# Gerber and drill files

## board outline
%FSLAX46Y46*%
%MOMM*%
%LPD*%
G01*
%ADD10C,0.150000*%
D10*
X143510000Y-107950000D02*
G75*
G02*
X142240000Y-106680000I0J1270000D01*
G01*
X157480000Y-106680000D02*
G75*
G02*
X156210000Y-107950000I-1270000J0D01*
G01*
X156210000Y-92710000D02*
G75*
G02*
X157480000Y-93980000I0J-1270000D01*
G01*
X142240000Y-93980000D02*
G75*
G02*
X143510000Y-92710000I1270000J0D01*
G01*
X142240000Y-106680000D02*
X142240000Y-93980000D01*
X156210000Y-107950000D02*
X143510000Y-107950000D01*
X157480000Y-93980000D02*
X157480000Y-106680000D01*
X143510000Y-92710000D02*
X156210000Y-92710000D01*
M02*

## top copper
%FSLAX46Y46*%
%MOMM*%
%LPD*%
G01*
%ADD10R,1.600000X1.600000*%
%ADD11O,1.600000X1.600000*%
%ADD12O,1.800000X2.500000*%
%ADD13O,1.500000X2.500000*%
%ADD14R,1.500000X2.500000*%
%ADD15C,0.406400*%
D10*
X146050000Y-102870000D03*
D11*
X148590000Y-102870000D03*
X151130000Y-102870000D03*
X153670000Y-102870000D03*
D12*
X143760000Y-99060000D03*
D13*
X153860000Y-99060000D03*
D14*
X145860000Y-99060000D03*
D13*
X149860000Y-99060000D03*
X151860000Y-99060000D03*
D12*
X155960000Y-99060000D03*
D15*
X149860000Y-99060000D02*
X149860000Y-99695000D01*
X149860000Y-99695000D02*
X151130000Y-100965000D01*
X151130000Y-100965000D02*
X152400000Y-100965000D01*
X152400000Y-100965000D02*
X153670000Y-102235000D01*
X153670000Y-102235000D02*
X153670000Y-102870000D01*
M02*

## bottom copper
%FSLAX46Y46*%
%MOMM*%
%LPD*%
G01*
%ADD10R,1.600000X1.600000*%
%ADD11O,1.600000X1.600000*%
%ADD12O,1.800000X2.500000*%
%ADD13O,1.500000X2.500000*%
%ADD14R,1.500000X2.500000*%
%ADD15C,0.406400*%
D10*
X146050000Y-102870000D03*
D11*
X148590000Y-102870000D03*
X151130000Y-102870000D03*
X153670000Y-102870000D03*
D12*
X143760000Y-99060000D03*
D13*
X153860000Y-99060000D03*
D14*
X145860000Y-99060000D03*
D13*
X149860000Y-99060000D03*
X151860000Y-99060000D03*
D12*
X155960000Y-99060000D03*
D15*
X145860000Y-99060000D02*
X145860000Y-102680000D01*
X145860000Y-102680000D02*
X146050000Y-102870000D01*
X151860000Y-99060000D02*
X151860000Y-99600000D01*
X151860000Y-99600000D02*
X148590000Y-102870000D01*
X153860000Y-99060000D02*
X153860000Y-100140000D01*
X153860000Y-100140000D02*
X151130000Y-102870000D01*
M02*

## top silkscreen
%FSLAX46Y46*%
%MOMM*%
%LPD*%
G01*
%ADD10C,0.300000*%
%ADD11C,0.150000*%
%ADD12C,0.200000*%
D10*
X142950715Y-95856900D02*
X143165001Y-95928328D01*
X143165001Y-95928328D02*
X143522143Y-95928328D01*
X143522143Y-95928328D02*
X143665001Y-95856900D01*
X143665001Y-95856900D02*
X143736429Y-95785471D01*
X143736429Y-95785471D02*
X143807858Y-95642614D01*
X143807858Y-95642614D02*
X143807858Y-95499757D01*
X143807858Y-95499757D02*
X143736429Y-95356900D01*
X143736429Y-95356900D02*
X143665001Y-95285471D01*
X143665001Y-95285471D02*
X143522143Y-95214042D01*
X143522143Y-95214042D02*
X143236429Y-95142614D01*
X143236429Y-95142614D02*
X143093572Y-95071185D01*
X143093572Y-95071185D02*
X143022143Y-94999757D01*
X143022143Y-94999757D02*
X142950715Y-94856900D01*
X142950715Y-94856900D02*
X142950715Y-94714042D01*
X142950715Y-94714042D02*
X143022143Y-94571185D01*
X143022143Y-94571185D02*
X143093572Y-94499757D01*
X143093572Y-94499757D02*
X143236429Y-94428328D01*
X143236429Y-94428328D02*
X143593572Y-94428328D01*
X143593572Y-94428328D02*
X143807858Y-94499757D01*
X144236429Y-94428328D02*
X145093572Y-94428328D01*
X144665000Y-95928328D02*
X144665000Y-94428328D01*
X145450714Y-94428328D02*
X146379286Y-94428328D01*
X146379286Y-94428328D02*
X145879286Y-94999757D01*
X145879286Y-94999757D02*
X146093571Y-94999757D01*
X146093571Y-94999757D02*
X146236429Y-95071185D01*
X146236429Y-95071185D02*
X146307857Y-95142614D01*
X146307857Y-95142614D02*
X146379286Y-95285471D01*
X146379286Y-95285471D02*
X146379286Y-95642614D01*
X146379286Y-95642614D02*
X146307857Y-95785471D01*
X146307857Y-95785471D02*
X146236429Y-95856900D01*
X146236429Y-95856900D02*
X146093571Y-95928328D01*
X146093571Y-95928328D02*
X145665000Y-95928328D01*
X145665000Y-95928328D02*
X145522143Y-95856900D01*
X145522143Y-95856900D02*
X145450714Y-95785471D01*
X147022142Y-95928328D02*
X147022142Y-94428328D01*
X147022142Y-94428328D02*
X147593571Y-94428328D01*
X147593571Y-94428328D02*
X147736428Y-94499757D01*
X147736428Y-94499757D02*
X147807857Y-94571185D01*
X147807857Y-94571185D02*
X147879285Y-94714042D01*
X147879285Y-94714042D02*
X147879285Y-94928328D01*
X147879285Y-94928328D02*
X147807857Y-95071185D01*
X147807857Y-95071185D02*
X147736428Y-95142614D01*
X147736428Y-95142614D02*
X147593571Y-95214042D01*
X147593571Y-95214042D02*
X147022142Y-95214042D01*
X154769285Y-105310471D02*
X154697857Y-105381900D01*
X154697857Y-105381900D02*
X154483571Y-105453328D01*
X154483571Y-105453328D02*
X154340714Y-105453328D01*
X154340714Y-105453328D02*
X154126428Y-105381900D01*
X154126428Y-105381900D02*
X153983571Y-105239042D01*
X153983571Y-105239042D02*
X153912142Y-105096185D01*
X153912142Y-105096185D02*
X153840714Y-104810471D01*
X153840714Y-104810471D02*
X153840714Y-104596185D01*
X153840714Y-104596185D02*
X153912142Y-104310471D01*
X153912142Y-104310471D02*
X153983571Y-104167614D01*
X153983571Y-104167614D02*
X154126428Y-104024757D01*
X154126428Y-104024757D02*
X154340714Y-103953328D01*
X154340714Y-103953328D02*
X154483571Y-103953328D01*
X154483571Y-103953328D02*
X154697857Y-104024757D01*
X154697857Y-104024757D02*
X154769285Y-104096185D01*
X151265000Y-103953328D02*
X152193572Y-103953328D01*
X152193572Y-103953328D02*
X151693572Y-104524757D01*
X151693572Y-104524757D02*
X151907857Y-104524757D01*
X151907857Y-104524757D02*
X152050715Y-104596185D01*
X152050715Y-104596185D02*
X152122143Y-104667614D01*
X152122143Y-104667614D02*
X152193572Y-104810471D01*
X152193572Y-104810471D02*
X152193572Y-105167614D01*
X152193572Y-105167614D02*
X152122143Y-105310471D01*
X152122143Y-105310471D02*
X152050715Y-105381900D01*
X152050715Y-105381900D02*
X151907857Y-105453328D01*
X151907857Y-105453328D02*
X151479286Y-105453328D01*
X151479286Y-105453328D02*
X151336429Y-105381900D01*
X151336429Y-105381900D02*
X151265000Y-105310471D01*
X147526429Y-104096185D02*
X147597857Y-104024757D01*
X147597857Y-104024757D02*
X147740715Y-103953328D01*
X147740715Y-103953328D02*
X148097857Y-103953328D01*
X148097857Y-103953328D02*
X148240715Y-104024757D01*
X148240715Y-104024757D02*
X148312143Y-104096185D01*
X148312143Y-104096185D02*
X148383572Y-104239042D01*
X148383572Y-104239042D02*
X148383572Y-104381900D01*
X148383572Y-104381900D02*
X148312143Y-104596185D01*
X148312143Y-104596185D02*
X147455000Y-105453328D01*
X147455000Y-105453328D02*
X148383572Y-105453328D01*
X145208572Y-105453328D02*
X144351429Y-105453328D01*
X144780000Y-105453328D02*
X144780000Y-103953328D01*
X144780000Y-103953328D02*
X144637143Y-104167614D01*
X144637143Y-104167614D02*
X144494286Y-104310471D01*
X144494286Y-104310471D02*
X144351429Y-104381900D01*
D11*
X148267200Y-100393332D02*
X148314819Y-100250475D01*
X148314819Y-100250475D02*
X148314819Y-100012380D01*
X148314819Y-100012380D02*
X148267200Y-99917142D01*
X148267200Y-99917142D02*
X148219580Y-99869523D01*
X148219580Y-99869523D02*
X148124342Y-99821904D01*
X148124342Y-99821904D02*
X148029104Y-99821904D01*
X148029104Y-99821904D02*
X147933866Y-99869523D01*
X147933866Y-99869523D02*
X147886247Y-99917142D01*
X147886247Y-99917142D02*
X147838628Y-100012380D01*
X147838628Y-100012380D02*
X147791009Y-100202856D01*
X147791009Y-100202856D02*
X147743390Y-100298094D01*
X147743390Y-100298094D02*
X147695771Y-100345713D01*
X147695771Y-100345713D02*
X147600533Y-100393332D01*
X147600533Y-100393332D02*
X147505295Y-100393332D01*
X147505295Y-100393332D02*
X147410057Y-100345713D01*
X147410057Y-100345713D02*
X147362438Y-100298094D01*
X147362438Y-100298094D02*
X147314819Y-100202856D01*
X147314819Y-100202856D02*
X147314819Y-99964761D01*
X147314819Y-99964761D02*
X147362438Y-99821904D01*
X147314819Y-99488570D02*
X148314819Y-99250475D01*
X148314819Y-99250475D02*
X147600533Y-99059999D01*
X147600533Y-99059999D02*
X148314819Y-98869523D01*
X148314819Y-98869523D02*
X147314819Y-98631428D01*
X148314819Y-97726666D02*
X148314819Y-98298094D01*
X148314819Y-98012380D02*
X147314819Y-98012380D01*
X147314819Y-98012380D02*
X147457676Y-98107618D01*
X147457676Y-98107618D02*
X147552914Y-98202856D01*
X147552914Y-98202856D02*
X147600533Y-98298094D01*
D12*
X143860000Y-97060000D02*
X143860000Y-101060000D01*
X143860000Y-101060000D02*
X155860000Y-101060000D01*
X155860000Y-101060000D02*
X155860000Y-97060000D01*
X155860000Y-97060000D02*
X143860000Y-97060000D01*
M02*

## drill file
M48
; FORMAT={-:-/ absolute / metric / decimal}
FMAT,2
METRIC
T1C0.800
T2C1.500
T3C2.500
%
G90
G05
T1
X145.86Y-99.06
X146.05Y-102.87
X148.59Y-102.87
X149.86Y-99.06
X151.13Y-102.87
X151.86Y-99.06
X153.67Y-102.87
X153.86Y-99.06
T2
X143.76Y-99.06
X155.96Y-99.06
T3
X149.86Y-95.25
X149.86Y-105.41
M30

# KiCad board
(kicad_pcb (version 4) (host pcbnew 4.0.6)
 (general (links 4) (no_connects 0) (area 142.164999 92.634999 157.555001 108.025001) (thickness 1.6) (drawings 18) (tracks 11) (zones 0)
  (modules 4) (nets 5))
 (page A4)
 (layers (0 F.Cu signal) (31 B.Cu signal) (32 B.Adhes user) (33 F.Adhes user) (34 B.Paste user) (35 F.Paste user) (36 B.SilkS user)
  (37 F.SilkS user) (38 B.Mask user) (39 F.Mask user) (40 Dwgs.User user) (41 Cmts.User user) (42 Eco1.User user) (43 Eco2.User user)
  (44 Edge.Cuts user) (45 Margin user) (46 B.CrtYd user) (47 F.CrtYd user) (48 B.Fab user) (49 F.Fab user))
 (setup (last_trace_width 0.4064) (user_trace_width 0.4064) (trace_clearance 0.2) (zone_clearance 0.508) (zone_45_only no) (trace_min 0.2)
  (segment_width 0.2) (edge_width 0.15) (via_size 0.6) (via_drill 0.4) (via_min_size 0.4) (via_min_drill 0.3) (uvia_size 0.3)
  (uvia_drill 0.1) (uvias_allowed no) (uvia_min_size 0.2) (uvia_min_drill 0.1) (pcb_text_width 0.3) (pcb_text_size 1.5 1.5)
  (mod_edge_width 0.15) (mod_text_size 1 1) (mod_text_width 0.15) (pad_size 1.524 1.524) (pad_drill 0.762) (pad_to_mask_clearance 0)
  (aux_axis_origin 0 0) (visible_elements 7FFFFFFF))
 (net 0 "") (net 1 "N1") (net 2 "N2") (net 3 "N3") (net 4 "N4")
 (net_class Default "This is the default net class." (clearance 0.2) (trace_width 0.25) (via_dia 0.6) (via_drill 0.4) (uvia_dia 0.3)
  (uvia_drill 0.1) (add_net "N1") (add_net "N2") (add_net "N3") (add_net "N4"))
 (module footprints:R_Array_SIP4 (layer F.Cu) (at 146.05 102.87)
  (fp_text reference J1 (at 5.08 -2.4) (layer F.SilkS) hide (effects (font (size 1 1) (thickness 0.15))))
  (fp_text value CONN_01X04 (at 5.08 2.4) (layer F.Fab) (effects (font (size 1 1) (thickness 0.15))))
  (pad 1 thru_hole rect (at 0 0) (size 1.6 1.6) (drill 0.8) (layers *.Cu *.Mask) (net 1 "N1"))
  (pad 2 thru_hole oval (at 2.54 0) (size 1.6 1.6) (drill 0.8) (layers *.Cu *.Mask) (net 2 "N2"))
  (pad 3 thru_hole oval (at 5.08 0) (size 1.6 1.6) (drill 0.8) (layers *.Cu *.Mask) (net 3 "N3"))
  (pad 4 thru_hole oval (at 7.62 0) (size 1.6 1.6) (drill 0.8) (layers *.Cu *.Mask) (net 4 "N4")))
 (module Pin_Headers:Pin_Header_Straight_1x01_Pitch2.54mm (layer F.Cu) (at 149.86 105.41)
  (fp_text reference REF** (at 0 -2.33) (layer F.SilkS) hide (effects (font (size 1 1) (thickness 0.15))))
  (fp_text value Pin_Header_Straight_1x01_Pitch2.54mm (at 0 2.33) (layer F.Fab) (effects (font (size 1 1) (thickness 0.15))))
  (pad "" np_thru_hole circle (at 0 0) (size 2.5 2.5) (drill 2.5) (layers *.Cu *.Mask)))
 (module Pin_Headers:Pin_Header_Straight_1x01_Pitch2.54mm (layer F.Cu) (at 149.86 95.25)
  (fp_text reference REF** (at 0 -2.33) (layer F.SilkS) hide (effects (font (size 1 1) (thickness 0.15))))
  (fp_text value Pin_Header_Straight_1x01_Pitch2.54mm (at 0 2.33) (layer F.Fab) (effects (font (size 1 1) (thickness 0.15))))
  (pad "" np_thru_hole circle (at 0 0) (size 2.5 2.5) (drill 2.5) (layers *.Cu *.Mask)))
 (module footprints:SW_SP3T (layer F.Cu) (at 149.86 99.06)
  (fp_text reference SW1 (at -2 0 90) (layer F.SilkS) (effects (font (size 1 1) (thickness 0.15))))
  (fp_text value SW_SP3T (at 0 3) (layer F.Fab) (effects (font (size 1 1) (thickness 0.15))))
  (fp_line (start -6 -2) (end -6 2) (layer F.SilkS) (width 0.2)) (fp_line (start -6 2) (end 6 2) (layer F.SilkS) (width 0.2))
  (fp_line (start 6 2) (end 6 -2) (layer F.SilkS) (width 0.2))
  (fp_line (start 6 -2) (end -6 -2) (layer F.SilkS) (width 0.2))
  (pad 5 thru_hole oval (at -6.1 0) (size 1.8 2.5) (drill 1.5) (layers *.Cu *.Mask))
  (pad 4 thru_hole oval (at 4 0) (size 1.5 2.5) (drill 0.8) (layers *.Cu *.Mask) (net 3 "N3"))
  (pad 1 thru_hole rect (at -4 0) (size 1.5 2.5) (drill 0.8) (layers *.Cu *.Mask) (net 1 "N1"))
  (pad 2 thru_hole oval (at 0 0) (size 1.5 2.5) (drill 0.8) (layers *.Cu *.Mask) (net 4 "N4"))
  (pad 3 thru_hole oval (at 2 0) (size 1.5 2.5) (drill 0.8) (layers *.Cu *.Mask) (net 2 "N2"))
  (pad 5 thru_hole oval (at 6.1 0) (size 1.8 2.5) (drill 1.5) (layers *.Cu *.Mask)))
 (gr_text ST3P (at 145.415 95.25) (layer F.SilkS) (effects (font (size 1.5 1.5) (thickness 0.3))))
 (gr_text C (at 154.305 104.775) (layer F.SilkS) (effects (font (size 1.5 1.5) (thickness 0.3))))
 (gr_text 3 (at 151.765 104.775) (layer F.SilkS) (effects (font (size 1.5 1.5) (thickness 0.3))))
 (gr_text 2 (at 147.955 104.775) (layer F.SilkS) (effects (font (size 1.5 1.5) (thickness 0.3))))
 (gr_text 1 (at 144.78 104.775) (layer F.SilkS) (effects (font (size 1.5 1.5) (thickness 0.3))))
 (gr_arc (start 143.51 106.68) (end 143.51 107.95) (angle 90) (layer Edge.Cuts) (width 0.15))
 (gr_arc (start 156.21 106.68) (end 157.48 106.68) (angle 90) (layer Edge.Cuts) (width 0.15))
 (gr_arc (start 156.21 93.98) (end 156.21 92.71) (angle 90) (layer Edge.Cuts) (width 0.15))
 (gr_arc (start 143.51 93.98) (end 142.24 93.98) (angle 90) (layer Edge.Cuts) (width 0.15))
 (gr_line (start 142.24 106.68) (end 142.24 93.98) (angle 90) (layer Edge.Cuts) (width 0.15))
 (gr_line (start 156.21 107.95) (end 143.51 107.95) (angle 90) (layer Edge.Cuts) (width 0.15))
 (gr_line (start 157.48 93.98) (end 157.48 106.68) (angle 90) (layer Edge.Cuts) (width 0.15))
 (gr_line (start 143.51 92.71) (end 156.21 92.71) (angle 90) (layer Edge.Cuts) (width 0.15))
 (segment (start 145.86 99.06) (end 145.86 102.68) (width 0.4064) (layer B.Cu) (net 1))
 (segment (start 145.86 102.68) (end 146.05 102.87) (width 0.4064) (layer B.Cu) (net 1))
 (segment (start 151.86 99.06) (end 151.86 99.6) (width 0.4064) (layer B.Cu) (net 2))
 (segment (start 151.86 99.6) (end 148.59 102.87) (width 0.4064) (layer B.Cu) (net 2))
 (segment (start 153.86 99.06) (end 153.86 100.14) (width 0.4064) (layer B.Cu) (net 3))
 (segment (start 153.86 100.14) (end 151.13 102.87) (width 0.4064) (layer B.Cu) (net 3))
 (segment (start 149.86 99.06) (end 149.86 99.695) (width 0.4064) (layer F.Cu) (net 4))
 (segment (start 149.86 99.695) (end 151.13 100.965) (width 0.4064) (layer F.Cu) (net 4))
 (segment (start 151.13 100.965) (end 152.4 100.965) (width 0.4064) (layer F.Cu) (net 4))
 (segment (start 152.4 100.965) (end 153.67 102.235) (width 0.4064) (layer F.Cu) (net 4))
 (segment (start 153.67 102.235) (end 153.67 102.87) (width 0.4064) (layer F.Cu) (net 4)))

